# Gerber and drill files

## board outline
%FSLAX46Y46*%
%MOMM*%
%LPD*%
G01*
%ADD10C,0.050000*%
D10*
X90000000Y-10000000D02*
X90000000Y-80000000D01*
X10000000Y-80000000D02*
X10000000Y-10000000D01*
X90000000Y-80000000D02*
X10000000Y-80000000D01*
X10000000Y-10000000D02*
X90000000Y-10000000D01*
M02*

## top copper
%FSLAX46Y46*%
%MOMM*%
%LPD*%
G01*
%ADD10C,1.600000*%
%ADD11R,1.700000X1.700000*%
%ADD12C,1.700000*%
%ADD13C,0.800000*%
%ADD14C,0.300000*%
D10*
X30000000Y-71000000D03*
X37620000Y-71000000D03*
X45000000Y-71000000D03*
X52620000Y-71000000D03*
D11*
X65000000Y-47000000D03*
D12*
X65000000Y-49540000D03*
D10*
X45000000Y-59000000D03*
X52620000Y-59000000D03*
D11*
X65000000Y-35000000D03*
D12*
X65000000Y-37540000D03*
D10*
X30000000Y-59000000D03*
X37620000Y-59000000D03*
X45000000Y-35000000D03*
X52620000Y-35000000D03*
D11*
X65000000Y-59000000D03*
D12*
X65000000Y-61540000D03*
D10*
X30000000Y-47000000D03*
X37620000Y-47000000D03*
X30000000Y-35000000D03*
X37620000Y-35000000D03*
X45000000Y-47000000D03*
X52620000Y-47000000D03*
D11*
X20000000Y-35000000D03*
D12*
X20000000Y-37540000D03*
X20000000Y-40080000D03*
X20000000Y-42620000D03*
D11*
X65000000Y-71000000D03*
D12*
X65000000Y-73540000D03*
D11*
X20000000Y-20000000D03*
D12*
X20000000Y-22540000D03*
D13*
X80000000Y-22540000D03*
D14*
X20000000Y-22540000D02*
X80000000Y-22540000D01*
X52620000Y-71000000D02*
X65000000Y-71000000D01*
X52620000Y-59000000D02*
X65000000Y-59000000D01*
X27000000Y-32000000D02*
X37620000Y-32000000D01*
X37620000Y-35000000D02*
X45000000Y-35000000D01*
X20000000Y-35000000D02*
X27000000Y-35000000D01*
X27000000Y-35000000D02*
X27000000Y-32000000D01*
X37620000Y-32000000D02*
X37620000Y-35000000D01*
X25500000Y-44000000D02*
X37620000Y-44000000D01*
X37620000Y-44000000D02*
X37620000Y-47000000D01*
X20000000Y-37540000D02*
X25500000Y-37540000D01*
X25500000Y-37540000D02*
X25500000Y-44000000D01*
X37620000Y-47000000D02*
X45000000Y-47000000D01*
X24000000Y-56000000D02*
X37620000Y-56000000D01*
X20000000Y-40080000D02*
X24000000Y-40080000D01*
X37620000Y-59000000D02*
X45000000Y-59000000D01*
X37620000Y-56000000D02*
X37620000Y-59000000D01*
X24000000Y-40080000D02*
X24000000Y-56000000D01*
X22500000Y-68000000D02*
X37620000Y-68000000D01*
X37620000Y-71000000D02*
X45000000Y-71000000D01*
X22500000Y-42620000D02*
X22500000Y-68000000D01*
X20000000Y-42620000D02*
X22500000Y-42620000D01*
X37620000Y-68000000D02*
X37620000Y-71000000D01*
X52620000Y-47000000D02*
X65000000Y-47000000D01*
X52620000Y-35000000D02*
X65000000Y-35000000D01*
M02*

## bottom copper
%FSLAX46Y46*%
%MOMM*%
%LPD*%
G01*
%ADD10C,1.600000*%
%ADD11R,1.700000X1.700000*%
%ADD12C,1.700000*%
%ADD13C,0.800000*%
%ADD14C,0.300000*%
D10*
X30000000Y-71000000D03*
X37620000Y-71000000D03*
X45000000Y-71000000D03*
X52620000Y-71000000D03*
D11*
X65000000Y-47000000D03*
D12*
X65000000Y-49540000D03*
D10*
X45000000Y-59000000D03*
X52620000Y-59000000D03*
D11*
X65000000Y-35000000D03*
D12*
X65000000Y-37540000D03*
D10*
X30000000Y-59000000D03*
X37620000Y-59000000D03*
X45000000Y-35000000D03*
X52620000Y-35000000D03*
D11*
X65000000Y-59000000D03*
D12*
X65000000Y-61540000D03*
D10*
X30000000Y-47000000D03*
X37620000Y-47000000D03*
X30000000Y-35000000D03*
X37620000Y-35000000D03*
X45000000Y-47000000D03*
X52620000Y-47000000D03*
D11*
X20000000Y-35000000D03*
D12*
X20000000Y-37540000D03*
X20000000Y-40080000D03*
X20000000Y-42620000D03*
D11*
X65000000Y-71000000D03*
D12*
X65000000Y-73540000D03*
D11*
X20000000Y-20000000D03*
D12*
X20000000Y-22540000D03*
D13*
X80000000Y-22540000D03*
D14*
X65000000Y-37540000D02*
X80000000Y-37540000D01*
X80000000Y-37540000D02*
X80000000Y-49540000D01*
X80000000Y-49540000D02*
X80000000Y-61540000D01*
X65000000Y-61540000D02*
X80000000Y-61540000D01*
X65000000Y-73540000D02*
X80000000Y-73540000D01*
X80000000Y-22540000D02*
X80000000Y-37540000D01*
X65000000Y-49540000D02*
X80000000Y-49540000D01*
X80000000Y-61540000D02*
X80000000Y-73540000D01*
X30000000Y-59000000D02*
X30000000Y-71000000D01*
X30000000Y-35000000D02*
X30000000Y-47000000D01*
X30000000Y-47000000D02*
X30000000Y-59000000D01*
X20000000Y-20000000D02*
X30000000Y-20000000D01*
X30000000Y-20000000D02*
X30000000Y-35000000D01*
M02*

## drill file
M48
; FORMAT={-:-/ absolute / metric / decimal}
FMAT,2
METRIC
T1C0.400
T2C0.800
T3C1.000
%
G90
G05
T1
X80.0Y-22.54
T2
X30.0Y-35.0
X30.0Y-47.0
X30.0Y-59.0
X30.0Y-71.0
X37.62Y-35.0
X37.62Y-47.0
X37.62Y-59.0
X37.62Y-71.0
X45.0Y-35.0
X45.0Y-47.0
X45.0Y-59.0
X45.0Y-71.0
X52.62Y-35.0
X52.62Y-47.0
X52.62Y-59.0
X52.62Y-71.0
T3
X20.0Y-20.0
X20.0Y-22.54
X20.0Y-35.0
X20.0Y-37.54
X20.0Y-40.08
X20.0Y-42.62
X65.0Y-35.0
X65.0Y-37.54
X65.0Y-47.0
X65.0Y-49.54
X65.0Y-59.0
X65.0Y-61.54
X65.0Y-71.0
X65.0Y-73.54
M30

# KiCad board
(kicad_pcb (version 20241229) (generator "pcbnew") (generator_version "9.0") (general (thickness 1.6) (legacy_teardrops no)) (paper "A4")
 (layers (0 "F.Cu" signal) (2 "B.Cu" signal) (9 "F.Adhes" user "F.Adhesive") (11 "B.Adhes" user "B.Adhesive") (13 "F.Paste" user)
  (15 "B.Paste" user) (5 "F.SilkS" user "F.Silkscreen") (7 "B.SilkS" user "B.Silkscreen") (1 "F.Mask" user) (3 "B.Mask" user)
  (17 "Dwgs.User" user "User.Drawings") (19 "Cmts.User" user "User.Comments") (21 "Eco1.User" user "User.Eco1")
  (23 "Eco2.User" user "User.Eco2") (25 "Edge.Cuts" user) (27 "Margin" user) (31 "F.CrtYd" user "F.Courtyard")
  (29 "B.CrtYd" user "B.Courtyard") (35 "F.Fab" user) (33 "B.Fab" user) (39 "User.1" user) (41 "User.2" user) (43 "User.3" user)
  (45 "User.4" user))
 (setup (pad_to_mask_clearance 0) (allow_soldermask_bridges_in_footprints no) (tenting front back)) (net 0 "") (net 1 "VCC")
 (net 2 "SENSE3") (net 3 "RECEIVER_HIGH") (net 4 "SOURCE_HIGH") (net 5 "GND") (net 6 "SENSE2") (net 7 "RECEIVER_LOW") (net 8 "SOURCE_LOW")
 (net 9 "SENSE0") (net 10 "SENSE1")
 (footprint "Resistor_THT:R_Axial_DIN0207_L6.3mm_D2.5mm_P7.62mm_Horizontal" (layer "F.Cu") (at 30 71)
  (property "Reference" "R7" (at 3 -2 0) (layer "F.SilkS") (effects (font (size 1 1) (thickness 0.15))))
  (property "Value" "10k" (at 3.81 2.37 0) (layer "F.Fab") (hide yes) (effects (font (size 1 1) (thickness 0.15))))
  (pad "1" thru_hole circle (at 0 0) (size 1.6 1.6) (drill 0.8) (layers "*.Cu" "*.Mask") (remove_unused_layers no) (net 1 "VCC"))
  (pad "2" thru_hole circle (at 7.62 0) (size 1.6 1.6) (drill 0.8) (layers "*.Cu" "*.Mask") (remove_unused_layers no) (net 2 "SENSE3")))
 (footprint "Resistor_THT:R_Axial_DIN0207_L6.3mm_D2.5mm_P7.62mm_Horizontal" (layer "F.Cu") (at 45 71)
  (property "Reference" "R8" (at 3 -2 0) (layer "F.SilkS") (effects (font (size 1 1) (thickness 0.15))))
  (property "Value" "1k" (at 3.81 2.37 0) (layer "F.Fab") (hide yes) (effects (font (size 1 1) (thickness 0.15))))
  (pad "1" thru_hole circle (at 0 0) (size 1.6 1.6) (drill 0.8) (layers "*.Cu" "*.Mask") (remove_unused_layers no) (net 2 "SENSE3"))
  (pad "2" thru_hole circle (at 7.62 0) (size 1.6 1.6) (drill 0.8) (layers "*.Cu" "*.Mask") (remove_unused_layers no)
   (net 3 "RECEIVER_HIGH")))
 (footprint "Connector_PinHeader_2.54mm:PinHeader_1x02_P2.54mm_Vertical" (layer "F.Cu") (at 65 47)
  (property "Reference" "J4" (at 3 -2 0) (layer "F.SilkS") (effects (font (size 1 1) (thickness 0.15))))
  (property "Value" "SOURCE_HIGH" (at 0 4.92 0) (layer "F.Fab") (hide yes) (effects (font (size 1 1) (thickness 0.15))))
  (pad "1" thru_hole rect (at 0 0) (size 1.7 1.7) (drill 1) (layers "*.Cu" "*.Mask") (remove_unused_layers no) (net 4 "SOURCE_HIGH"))
  (pad "2" thru_hole circle (at 0 2.54) (size 1.7 1.7) (drill 1) (layers "*.Cu" "*.Mask") (remove_unused_layers no) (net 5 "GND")))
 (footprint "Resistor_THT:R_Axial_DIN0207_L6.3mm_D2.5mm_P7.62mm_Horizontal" (layer "F.Cu") (at 45 59)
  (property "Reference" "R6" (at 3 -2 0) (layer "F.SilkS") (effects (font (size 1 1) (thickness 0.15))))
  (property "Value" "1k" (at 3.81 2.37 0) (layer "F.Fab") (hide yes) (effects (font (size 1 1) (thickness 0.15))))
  (pad "1" thru_hole circle (at 0 0) (size 1.6 1.6) (drill 0.8) (layers "*.Cu" "*.Mask") (remove_unused_layers no) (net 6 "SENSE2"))
  (pad "2" thru_hole circle (at 7.62 0) (size 1.6 1.6) (drill 0.8) (layers "*.Cu" "*.Mask") (remove_unused_layers no) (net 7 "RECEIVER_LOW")))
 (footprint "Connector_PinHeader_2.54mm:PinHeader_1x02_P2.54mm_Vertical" (layer "F.Cu") (at 65 35)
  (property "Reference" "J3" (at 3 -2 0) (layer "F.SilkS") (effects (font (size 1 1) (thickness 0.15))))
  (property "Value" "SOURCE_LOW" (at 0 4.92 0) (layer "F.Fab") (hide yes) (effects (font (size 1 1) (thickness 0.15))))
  (pad "1" thru_hole rect (at 0 0) (size 1.7 1.7) (drill 1) (layers "*.Cu" "*.Mask") (remove_unused_layers no) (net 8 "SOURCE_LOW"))
  (pad "2" thru_hole circle (at 0 2.54) (size 1.7 1.7) (drill 1) (layers "*.Cu" "*.Mask") (remove_unused_layers no) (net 5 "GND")))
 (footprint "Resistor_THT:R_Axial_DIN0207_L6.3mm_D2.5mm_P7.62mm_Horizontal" (layer "F.Cu") (at 30 59)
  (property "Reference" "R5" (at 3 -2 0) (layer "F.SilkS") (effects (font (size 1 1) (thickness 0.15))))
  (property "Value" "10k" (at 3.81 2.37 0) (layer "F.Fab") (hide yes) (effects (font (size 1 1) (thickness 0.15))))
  (pad "1" thru_hole circle (at 0 0) (size 1.6 1.6) (drill 0.8) (layers "*.Cu" "*.Mask") (remove_unused_layers no) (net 1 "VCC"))
  (pad "2" thru_hole circle (at 7.62 0) (size 1.6 1.6) (drill 0.8) (layers "*.Cu" "*.Mask") (remove_unused_layers no) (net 6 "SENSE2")))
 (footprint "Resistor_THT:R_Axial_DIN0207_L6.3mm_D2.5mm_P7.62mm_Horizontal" (layer "F.Cu") (at 45 35)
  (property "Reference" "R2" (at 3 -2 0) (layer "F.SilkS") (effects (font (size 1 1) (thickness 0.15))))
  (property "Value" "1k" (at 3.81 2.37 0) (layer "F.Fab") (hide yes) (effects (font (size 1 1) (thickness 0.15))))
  (pad "1" thru_hole circle (at 0 0) (size 1.6 1.6) (drill 0.8) (layers "*.Cu" "*.Mask") (remove_unused_layers no) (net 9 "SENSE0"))
  (pad "2" thru_hole circle (at 7.62 0) (size 1.6 1.6) (drill 0.8) (layers "*.Cu" "*.Mask") (remove_unused_layers no) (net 8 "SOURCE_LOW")))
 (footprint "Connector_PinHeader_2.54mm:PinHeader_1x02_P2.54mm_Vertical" (layer "F.Cu") (at 65 59)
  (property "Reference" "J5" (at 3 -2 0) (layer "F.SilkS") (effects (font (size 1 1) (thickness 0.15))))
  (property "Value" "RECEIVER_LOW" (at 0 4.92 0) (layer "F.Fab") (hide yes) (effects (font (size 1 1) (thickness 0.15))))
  (pad "1" thru_hole rect (at 0 0) (size 1.7 1.7) (drill 1) (layers "*.Cu" "*.Mask") (remove_unused_layers no) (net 7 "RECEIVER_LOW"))
  (pad "2" thru_hole circle (at 0 2.54) (size 1.7 1.7) (drill 1) (layers "*.Cu" "*.Mask") (remove_unused_layers no) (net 5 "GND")))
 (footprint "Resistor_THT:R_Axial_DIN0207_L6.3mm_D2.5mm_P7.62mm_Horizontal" (layer "F.Cu") (at 30 47)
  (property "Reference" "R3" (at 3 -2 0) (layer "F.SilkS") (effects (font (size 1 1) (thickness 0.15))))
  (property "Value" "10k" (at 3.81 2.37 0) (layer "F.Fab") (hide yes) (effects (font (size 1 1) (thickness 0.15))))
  (pad "1" thru_hole circle (at 0 0) (size 1.6 1.6) (drill 0.8) (layers "*.Cu" "*.Mask") (remove_unused_layers no) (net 1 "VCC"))
  (pad "2" thru_hole circle (at 7.62 0) (size 1.6 1.6) (drill 0.8) (layers "*.Cu" "*.Mask") (remove_unused_layers no) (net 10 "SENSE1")))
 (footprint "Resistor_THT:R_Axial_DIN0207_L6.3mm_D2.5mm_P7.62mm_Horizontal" (layer "F.Cu") (at 30 35)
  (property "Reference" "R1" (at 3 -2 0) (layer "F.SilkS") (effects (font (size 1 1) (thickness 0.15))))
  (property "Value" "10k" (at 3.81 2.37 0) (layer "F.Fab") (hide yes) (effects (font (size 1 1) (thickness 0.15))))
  (pad "1" thru_hole circle (at 0 0) (size 1.6 1.6) (drill 0.8) (layers "*.Cu" "*.Mask") (remove_unused_layers no) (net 1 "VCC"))
  (pad "2" thru_hole circle (at 7.62 0) (size 1.6 1.6) (drill 0.8) (layers "*.Cu" "*.Mask") (remove_unused_layers no) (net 9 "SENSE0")))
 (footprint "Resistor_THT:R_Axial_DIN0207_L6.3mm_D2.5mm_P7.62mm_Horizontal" (layer "F.Cu") (at 45 47)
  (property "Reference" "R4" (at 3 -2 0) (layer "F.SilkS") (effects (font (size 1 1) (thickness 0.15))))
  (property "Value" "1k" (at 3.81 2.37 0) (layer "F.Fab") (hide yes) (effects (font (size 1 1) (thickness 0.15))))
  (pad "1" thru_hole circle (at 0 0) (size 1.6 1.6) (drill 0.8) (layers "*.Cu" "*.Mask") (remove_unused_layers no) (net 10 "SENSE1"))
  (pad "2" thru_hole circle (at 7.62 0) (size 1.6 1.6) (drill 0.8) (layers "*.Cu" "*.Mask") (remove_unused_layers no) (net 4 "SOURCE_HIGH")))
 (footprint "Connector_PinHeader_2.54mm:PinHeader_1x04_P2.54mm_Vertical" (layer "F.Cu") (at 20 35)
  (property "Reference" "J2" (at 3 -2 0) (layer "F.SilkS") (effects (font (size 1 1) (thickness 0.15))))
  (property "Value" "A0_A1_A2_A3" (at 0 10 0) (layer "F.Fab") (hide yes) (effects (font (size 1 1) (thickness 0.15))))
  (pad "1" thru_hole rect (at 0 0) (size 1.7 1.7) (drill 1) (layers "*.Cu" "*.Mask") (remove_unused_layers no) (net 9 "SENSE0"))
  (pad "2" thru_hole circle (at 0 2.54) (size 1.7 1.7) (drill 1) (layers "*.Cu" "*.Mask") (remove_unused_layers no) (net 10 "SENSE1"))
  (pad "3" thru_hole circle (at 0 5.08) (size 1.7 1.7) (drill 1) (layers "*.Cu" "*.Mask") (remove_unused_layers no) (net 6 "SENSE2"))
  (pad "4" thru_hole circle (at 0 7.62) (size 1.7 1.7) (drill 1) (layers "*.Cu" "*.Mask") (remove_unused_layers no) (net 2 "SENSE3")))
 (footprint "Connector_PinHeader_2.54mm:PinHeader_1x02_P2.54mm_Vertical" (layer "F.Cu") (at 65 71)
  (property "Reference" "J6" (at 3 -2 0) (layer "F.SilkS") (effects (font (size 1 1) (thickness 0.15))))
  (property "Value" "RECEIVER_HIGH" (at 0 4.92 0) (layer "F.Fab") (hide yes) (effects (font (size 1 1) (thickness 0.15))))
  (pad "1" thru_hole rect (at 0 0) (size 1.7 1.7) (drill 1) (layers "*.Cu" "*.Mask") (remove_unused_layers no) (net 3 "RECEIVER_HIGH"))
  (pad "2" thru_hole circle (at 0 2.54) (size 1.7 1.7) (drill 1) (layers "*.Cu" "*.Mask") (remove_unused_layers no) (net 5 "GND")))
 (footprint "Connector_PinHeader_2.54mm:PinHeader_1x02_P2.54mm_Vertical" (layer "F.Cu") (at 20 20)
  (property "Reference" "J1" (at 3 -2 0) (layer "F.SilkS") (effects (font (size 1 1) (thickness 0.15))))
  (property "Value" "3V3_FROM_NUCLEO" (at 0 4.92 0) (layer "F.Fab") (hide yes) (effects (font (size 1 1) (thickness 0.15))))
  (pad "1" thru_hole rect (at 0 0) (size 1.7 1.7) (drill 1) (layers "*.Cu" "*.Mask") (remove_unused_layers no) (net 1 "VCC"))
  (pad "2" thru_hole circle (at 0 2.54) (size 1.7 1.7) (drill 1) (layers "*.Cu" "*.Mask") (remove_unused_layers no) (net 5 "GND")))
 (gr_line (start 90 10) (end 90 80) (stroke (width 0.05) (type default)) (layer "Edge.Cuts"))
 (gr_line (start 10 80) (end 10 10) (stroke (width 0.05) (type default)) (layer "Edge.Cuts"))
 (gr_line (start 90 80) (end 10 80) (stroke (width 0.05) (type default)) (layer "Edge.Cuts"))
 (gr_line (start 10 10) (end 90 10) (stroke (width 0.05) (type default)) (layer "Edge.Cuts"))
 (segment (start 20 22.54) (end 80 22.54) (width 0.3) (layer "F.Cu") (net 5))
 (via (at 80 22.54) (size 0.8) (drill 0.4) (layers "F.Cu" "B.Cu") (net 5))
 (segment (start 65 37.54) (end 80 37.54) (width 0.3) (layer "B.Cu") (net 5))
 (segment (start 80 37.54) (end 80 49.54) (width 0.3) (layer "B.Cu") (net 5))
 (segment (start 80 49.54) (end 80 61.54) (width 0.3) (layer "B.Cu") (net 5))
 (segment (start 65 61.54) (end 80 61.54) (width 0.3) (layer "B.Cu") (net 5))
 (segment (start 65 73.54) (end 80 73.54) (width 0.3) (layer "B.Cu") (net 5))
 (segment (start 80 22.54) (end 80 37.54) (width 0.3) (layer "B.Cu") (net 5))
 (segment (start 65 49.54) (end 80 49.54) (width 0.3) (layer "B.Cu") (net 5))
 (segment (start 80 61.54) (end 80 73.54) (width 0.3) (layer "B.Cu") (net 5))
 (segment (start 52.62 71) (end 65 71) (width 0.3) (layer "F.Cu") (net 3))
 (segment (start 52.62 59) (end 65 59) (width 0.3) (layer "F.Cu") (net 7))
 (segment (start 27 32) (end 37.62 32) (width 0.3) (layer "F.Cu") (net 9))
 (segment (start 37.62 35) (end 45 35) (width 0.3) (layer "F.Cu") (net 9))
 (segment (start 20 35) (end 27 35) (width 0.3) (layer "F.Cu") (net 9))
 (segment (start 27 35) (end 27 32) (width 0.3) (layer "F.Cu") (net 9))
 (segment (start 37.62 32) (end 37.62 35) (width 0.3) (layer "F.Cu") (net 9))
 (segment (start 25.5 44) (end 37.62 44) (width 0.3) (layer "F.Cu") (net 10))
 (segment (start 37.62 44) (end 37.62 47) (width 0.3) (layer "F.Cu") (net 10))
 (segment (start 20 37.54) (end 25.5 37.54) (width 0.3) (layer "F.Cu") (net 10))
 (segment (start 25.5 37.54) (end 25.5 44) (width 0.3) (layer "F.Cu") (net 10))
 (segment (start 37.62 47) (end 45 47) (width 0.3) (layer "F.Cu") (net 10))
 (segment (start 24 56) (end 37.62 56) (width 0.3) (layer "F.Cu") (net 6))
 (segment (start 20 40.08) (end 24 40.08) (width 0.3) (layer "F.Cu") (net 6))
 (segment (start 37.62 59) (end 45 59) (width 0.3) (layer "F.Cu") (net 6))
 (segment (start 37.62 56) (end 37.62 59) (width 0.3) (layer "F.Cu") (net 6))
 (segment (start 24 40.08) (end 24 56) (width 0.3) (layer "F.Cu") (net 6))
 (segment (start 22.5 68) (end 37.62 68) (width 0.3) (layer "F.Cu") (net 2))
 (segment (start 37.62 71) (end 45 71) (width 0.3) (layer "F.Cu") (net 2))
 (segment (start 22.5 42.62) (end 22.5 68) (width 0.3) (layer "F.Cu") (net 2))
 (segment (start 20 42.62) (end 22.5 42.62) (width 0.3) (layer "F.Cu") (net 2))
 (segment (start 37.62 68) (end 37.62 71) (width 0.3) (layer "F.Cu") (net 2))
 (segment (start 52.62 47) (end 65 47) (width 0.3) (layer "F.Cu") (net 4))
 (segment (start 52.62 35) (end 65 35) (width 0.3) (layer "F.Cu") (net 8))
 (segment (start 30 59) (end 30 71) (width 0.3) (layer "B.Cu") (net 1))
 (segment (start 30 35) (end 30 47) (width 0.3) (layer "B.Cu") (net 1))
 (segment (start 30 47) (end 30 59) (width 0.3) (layer "B.Cu") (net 1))
 (segment (start 20 20) (end 30 20) (width 0.3) (layer "B.Cu") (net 1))
 (segment (start 30 20) (end 30 35) (width 0.3) (layer "B.Cu") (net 1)))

